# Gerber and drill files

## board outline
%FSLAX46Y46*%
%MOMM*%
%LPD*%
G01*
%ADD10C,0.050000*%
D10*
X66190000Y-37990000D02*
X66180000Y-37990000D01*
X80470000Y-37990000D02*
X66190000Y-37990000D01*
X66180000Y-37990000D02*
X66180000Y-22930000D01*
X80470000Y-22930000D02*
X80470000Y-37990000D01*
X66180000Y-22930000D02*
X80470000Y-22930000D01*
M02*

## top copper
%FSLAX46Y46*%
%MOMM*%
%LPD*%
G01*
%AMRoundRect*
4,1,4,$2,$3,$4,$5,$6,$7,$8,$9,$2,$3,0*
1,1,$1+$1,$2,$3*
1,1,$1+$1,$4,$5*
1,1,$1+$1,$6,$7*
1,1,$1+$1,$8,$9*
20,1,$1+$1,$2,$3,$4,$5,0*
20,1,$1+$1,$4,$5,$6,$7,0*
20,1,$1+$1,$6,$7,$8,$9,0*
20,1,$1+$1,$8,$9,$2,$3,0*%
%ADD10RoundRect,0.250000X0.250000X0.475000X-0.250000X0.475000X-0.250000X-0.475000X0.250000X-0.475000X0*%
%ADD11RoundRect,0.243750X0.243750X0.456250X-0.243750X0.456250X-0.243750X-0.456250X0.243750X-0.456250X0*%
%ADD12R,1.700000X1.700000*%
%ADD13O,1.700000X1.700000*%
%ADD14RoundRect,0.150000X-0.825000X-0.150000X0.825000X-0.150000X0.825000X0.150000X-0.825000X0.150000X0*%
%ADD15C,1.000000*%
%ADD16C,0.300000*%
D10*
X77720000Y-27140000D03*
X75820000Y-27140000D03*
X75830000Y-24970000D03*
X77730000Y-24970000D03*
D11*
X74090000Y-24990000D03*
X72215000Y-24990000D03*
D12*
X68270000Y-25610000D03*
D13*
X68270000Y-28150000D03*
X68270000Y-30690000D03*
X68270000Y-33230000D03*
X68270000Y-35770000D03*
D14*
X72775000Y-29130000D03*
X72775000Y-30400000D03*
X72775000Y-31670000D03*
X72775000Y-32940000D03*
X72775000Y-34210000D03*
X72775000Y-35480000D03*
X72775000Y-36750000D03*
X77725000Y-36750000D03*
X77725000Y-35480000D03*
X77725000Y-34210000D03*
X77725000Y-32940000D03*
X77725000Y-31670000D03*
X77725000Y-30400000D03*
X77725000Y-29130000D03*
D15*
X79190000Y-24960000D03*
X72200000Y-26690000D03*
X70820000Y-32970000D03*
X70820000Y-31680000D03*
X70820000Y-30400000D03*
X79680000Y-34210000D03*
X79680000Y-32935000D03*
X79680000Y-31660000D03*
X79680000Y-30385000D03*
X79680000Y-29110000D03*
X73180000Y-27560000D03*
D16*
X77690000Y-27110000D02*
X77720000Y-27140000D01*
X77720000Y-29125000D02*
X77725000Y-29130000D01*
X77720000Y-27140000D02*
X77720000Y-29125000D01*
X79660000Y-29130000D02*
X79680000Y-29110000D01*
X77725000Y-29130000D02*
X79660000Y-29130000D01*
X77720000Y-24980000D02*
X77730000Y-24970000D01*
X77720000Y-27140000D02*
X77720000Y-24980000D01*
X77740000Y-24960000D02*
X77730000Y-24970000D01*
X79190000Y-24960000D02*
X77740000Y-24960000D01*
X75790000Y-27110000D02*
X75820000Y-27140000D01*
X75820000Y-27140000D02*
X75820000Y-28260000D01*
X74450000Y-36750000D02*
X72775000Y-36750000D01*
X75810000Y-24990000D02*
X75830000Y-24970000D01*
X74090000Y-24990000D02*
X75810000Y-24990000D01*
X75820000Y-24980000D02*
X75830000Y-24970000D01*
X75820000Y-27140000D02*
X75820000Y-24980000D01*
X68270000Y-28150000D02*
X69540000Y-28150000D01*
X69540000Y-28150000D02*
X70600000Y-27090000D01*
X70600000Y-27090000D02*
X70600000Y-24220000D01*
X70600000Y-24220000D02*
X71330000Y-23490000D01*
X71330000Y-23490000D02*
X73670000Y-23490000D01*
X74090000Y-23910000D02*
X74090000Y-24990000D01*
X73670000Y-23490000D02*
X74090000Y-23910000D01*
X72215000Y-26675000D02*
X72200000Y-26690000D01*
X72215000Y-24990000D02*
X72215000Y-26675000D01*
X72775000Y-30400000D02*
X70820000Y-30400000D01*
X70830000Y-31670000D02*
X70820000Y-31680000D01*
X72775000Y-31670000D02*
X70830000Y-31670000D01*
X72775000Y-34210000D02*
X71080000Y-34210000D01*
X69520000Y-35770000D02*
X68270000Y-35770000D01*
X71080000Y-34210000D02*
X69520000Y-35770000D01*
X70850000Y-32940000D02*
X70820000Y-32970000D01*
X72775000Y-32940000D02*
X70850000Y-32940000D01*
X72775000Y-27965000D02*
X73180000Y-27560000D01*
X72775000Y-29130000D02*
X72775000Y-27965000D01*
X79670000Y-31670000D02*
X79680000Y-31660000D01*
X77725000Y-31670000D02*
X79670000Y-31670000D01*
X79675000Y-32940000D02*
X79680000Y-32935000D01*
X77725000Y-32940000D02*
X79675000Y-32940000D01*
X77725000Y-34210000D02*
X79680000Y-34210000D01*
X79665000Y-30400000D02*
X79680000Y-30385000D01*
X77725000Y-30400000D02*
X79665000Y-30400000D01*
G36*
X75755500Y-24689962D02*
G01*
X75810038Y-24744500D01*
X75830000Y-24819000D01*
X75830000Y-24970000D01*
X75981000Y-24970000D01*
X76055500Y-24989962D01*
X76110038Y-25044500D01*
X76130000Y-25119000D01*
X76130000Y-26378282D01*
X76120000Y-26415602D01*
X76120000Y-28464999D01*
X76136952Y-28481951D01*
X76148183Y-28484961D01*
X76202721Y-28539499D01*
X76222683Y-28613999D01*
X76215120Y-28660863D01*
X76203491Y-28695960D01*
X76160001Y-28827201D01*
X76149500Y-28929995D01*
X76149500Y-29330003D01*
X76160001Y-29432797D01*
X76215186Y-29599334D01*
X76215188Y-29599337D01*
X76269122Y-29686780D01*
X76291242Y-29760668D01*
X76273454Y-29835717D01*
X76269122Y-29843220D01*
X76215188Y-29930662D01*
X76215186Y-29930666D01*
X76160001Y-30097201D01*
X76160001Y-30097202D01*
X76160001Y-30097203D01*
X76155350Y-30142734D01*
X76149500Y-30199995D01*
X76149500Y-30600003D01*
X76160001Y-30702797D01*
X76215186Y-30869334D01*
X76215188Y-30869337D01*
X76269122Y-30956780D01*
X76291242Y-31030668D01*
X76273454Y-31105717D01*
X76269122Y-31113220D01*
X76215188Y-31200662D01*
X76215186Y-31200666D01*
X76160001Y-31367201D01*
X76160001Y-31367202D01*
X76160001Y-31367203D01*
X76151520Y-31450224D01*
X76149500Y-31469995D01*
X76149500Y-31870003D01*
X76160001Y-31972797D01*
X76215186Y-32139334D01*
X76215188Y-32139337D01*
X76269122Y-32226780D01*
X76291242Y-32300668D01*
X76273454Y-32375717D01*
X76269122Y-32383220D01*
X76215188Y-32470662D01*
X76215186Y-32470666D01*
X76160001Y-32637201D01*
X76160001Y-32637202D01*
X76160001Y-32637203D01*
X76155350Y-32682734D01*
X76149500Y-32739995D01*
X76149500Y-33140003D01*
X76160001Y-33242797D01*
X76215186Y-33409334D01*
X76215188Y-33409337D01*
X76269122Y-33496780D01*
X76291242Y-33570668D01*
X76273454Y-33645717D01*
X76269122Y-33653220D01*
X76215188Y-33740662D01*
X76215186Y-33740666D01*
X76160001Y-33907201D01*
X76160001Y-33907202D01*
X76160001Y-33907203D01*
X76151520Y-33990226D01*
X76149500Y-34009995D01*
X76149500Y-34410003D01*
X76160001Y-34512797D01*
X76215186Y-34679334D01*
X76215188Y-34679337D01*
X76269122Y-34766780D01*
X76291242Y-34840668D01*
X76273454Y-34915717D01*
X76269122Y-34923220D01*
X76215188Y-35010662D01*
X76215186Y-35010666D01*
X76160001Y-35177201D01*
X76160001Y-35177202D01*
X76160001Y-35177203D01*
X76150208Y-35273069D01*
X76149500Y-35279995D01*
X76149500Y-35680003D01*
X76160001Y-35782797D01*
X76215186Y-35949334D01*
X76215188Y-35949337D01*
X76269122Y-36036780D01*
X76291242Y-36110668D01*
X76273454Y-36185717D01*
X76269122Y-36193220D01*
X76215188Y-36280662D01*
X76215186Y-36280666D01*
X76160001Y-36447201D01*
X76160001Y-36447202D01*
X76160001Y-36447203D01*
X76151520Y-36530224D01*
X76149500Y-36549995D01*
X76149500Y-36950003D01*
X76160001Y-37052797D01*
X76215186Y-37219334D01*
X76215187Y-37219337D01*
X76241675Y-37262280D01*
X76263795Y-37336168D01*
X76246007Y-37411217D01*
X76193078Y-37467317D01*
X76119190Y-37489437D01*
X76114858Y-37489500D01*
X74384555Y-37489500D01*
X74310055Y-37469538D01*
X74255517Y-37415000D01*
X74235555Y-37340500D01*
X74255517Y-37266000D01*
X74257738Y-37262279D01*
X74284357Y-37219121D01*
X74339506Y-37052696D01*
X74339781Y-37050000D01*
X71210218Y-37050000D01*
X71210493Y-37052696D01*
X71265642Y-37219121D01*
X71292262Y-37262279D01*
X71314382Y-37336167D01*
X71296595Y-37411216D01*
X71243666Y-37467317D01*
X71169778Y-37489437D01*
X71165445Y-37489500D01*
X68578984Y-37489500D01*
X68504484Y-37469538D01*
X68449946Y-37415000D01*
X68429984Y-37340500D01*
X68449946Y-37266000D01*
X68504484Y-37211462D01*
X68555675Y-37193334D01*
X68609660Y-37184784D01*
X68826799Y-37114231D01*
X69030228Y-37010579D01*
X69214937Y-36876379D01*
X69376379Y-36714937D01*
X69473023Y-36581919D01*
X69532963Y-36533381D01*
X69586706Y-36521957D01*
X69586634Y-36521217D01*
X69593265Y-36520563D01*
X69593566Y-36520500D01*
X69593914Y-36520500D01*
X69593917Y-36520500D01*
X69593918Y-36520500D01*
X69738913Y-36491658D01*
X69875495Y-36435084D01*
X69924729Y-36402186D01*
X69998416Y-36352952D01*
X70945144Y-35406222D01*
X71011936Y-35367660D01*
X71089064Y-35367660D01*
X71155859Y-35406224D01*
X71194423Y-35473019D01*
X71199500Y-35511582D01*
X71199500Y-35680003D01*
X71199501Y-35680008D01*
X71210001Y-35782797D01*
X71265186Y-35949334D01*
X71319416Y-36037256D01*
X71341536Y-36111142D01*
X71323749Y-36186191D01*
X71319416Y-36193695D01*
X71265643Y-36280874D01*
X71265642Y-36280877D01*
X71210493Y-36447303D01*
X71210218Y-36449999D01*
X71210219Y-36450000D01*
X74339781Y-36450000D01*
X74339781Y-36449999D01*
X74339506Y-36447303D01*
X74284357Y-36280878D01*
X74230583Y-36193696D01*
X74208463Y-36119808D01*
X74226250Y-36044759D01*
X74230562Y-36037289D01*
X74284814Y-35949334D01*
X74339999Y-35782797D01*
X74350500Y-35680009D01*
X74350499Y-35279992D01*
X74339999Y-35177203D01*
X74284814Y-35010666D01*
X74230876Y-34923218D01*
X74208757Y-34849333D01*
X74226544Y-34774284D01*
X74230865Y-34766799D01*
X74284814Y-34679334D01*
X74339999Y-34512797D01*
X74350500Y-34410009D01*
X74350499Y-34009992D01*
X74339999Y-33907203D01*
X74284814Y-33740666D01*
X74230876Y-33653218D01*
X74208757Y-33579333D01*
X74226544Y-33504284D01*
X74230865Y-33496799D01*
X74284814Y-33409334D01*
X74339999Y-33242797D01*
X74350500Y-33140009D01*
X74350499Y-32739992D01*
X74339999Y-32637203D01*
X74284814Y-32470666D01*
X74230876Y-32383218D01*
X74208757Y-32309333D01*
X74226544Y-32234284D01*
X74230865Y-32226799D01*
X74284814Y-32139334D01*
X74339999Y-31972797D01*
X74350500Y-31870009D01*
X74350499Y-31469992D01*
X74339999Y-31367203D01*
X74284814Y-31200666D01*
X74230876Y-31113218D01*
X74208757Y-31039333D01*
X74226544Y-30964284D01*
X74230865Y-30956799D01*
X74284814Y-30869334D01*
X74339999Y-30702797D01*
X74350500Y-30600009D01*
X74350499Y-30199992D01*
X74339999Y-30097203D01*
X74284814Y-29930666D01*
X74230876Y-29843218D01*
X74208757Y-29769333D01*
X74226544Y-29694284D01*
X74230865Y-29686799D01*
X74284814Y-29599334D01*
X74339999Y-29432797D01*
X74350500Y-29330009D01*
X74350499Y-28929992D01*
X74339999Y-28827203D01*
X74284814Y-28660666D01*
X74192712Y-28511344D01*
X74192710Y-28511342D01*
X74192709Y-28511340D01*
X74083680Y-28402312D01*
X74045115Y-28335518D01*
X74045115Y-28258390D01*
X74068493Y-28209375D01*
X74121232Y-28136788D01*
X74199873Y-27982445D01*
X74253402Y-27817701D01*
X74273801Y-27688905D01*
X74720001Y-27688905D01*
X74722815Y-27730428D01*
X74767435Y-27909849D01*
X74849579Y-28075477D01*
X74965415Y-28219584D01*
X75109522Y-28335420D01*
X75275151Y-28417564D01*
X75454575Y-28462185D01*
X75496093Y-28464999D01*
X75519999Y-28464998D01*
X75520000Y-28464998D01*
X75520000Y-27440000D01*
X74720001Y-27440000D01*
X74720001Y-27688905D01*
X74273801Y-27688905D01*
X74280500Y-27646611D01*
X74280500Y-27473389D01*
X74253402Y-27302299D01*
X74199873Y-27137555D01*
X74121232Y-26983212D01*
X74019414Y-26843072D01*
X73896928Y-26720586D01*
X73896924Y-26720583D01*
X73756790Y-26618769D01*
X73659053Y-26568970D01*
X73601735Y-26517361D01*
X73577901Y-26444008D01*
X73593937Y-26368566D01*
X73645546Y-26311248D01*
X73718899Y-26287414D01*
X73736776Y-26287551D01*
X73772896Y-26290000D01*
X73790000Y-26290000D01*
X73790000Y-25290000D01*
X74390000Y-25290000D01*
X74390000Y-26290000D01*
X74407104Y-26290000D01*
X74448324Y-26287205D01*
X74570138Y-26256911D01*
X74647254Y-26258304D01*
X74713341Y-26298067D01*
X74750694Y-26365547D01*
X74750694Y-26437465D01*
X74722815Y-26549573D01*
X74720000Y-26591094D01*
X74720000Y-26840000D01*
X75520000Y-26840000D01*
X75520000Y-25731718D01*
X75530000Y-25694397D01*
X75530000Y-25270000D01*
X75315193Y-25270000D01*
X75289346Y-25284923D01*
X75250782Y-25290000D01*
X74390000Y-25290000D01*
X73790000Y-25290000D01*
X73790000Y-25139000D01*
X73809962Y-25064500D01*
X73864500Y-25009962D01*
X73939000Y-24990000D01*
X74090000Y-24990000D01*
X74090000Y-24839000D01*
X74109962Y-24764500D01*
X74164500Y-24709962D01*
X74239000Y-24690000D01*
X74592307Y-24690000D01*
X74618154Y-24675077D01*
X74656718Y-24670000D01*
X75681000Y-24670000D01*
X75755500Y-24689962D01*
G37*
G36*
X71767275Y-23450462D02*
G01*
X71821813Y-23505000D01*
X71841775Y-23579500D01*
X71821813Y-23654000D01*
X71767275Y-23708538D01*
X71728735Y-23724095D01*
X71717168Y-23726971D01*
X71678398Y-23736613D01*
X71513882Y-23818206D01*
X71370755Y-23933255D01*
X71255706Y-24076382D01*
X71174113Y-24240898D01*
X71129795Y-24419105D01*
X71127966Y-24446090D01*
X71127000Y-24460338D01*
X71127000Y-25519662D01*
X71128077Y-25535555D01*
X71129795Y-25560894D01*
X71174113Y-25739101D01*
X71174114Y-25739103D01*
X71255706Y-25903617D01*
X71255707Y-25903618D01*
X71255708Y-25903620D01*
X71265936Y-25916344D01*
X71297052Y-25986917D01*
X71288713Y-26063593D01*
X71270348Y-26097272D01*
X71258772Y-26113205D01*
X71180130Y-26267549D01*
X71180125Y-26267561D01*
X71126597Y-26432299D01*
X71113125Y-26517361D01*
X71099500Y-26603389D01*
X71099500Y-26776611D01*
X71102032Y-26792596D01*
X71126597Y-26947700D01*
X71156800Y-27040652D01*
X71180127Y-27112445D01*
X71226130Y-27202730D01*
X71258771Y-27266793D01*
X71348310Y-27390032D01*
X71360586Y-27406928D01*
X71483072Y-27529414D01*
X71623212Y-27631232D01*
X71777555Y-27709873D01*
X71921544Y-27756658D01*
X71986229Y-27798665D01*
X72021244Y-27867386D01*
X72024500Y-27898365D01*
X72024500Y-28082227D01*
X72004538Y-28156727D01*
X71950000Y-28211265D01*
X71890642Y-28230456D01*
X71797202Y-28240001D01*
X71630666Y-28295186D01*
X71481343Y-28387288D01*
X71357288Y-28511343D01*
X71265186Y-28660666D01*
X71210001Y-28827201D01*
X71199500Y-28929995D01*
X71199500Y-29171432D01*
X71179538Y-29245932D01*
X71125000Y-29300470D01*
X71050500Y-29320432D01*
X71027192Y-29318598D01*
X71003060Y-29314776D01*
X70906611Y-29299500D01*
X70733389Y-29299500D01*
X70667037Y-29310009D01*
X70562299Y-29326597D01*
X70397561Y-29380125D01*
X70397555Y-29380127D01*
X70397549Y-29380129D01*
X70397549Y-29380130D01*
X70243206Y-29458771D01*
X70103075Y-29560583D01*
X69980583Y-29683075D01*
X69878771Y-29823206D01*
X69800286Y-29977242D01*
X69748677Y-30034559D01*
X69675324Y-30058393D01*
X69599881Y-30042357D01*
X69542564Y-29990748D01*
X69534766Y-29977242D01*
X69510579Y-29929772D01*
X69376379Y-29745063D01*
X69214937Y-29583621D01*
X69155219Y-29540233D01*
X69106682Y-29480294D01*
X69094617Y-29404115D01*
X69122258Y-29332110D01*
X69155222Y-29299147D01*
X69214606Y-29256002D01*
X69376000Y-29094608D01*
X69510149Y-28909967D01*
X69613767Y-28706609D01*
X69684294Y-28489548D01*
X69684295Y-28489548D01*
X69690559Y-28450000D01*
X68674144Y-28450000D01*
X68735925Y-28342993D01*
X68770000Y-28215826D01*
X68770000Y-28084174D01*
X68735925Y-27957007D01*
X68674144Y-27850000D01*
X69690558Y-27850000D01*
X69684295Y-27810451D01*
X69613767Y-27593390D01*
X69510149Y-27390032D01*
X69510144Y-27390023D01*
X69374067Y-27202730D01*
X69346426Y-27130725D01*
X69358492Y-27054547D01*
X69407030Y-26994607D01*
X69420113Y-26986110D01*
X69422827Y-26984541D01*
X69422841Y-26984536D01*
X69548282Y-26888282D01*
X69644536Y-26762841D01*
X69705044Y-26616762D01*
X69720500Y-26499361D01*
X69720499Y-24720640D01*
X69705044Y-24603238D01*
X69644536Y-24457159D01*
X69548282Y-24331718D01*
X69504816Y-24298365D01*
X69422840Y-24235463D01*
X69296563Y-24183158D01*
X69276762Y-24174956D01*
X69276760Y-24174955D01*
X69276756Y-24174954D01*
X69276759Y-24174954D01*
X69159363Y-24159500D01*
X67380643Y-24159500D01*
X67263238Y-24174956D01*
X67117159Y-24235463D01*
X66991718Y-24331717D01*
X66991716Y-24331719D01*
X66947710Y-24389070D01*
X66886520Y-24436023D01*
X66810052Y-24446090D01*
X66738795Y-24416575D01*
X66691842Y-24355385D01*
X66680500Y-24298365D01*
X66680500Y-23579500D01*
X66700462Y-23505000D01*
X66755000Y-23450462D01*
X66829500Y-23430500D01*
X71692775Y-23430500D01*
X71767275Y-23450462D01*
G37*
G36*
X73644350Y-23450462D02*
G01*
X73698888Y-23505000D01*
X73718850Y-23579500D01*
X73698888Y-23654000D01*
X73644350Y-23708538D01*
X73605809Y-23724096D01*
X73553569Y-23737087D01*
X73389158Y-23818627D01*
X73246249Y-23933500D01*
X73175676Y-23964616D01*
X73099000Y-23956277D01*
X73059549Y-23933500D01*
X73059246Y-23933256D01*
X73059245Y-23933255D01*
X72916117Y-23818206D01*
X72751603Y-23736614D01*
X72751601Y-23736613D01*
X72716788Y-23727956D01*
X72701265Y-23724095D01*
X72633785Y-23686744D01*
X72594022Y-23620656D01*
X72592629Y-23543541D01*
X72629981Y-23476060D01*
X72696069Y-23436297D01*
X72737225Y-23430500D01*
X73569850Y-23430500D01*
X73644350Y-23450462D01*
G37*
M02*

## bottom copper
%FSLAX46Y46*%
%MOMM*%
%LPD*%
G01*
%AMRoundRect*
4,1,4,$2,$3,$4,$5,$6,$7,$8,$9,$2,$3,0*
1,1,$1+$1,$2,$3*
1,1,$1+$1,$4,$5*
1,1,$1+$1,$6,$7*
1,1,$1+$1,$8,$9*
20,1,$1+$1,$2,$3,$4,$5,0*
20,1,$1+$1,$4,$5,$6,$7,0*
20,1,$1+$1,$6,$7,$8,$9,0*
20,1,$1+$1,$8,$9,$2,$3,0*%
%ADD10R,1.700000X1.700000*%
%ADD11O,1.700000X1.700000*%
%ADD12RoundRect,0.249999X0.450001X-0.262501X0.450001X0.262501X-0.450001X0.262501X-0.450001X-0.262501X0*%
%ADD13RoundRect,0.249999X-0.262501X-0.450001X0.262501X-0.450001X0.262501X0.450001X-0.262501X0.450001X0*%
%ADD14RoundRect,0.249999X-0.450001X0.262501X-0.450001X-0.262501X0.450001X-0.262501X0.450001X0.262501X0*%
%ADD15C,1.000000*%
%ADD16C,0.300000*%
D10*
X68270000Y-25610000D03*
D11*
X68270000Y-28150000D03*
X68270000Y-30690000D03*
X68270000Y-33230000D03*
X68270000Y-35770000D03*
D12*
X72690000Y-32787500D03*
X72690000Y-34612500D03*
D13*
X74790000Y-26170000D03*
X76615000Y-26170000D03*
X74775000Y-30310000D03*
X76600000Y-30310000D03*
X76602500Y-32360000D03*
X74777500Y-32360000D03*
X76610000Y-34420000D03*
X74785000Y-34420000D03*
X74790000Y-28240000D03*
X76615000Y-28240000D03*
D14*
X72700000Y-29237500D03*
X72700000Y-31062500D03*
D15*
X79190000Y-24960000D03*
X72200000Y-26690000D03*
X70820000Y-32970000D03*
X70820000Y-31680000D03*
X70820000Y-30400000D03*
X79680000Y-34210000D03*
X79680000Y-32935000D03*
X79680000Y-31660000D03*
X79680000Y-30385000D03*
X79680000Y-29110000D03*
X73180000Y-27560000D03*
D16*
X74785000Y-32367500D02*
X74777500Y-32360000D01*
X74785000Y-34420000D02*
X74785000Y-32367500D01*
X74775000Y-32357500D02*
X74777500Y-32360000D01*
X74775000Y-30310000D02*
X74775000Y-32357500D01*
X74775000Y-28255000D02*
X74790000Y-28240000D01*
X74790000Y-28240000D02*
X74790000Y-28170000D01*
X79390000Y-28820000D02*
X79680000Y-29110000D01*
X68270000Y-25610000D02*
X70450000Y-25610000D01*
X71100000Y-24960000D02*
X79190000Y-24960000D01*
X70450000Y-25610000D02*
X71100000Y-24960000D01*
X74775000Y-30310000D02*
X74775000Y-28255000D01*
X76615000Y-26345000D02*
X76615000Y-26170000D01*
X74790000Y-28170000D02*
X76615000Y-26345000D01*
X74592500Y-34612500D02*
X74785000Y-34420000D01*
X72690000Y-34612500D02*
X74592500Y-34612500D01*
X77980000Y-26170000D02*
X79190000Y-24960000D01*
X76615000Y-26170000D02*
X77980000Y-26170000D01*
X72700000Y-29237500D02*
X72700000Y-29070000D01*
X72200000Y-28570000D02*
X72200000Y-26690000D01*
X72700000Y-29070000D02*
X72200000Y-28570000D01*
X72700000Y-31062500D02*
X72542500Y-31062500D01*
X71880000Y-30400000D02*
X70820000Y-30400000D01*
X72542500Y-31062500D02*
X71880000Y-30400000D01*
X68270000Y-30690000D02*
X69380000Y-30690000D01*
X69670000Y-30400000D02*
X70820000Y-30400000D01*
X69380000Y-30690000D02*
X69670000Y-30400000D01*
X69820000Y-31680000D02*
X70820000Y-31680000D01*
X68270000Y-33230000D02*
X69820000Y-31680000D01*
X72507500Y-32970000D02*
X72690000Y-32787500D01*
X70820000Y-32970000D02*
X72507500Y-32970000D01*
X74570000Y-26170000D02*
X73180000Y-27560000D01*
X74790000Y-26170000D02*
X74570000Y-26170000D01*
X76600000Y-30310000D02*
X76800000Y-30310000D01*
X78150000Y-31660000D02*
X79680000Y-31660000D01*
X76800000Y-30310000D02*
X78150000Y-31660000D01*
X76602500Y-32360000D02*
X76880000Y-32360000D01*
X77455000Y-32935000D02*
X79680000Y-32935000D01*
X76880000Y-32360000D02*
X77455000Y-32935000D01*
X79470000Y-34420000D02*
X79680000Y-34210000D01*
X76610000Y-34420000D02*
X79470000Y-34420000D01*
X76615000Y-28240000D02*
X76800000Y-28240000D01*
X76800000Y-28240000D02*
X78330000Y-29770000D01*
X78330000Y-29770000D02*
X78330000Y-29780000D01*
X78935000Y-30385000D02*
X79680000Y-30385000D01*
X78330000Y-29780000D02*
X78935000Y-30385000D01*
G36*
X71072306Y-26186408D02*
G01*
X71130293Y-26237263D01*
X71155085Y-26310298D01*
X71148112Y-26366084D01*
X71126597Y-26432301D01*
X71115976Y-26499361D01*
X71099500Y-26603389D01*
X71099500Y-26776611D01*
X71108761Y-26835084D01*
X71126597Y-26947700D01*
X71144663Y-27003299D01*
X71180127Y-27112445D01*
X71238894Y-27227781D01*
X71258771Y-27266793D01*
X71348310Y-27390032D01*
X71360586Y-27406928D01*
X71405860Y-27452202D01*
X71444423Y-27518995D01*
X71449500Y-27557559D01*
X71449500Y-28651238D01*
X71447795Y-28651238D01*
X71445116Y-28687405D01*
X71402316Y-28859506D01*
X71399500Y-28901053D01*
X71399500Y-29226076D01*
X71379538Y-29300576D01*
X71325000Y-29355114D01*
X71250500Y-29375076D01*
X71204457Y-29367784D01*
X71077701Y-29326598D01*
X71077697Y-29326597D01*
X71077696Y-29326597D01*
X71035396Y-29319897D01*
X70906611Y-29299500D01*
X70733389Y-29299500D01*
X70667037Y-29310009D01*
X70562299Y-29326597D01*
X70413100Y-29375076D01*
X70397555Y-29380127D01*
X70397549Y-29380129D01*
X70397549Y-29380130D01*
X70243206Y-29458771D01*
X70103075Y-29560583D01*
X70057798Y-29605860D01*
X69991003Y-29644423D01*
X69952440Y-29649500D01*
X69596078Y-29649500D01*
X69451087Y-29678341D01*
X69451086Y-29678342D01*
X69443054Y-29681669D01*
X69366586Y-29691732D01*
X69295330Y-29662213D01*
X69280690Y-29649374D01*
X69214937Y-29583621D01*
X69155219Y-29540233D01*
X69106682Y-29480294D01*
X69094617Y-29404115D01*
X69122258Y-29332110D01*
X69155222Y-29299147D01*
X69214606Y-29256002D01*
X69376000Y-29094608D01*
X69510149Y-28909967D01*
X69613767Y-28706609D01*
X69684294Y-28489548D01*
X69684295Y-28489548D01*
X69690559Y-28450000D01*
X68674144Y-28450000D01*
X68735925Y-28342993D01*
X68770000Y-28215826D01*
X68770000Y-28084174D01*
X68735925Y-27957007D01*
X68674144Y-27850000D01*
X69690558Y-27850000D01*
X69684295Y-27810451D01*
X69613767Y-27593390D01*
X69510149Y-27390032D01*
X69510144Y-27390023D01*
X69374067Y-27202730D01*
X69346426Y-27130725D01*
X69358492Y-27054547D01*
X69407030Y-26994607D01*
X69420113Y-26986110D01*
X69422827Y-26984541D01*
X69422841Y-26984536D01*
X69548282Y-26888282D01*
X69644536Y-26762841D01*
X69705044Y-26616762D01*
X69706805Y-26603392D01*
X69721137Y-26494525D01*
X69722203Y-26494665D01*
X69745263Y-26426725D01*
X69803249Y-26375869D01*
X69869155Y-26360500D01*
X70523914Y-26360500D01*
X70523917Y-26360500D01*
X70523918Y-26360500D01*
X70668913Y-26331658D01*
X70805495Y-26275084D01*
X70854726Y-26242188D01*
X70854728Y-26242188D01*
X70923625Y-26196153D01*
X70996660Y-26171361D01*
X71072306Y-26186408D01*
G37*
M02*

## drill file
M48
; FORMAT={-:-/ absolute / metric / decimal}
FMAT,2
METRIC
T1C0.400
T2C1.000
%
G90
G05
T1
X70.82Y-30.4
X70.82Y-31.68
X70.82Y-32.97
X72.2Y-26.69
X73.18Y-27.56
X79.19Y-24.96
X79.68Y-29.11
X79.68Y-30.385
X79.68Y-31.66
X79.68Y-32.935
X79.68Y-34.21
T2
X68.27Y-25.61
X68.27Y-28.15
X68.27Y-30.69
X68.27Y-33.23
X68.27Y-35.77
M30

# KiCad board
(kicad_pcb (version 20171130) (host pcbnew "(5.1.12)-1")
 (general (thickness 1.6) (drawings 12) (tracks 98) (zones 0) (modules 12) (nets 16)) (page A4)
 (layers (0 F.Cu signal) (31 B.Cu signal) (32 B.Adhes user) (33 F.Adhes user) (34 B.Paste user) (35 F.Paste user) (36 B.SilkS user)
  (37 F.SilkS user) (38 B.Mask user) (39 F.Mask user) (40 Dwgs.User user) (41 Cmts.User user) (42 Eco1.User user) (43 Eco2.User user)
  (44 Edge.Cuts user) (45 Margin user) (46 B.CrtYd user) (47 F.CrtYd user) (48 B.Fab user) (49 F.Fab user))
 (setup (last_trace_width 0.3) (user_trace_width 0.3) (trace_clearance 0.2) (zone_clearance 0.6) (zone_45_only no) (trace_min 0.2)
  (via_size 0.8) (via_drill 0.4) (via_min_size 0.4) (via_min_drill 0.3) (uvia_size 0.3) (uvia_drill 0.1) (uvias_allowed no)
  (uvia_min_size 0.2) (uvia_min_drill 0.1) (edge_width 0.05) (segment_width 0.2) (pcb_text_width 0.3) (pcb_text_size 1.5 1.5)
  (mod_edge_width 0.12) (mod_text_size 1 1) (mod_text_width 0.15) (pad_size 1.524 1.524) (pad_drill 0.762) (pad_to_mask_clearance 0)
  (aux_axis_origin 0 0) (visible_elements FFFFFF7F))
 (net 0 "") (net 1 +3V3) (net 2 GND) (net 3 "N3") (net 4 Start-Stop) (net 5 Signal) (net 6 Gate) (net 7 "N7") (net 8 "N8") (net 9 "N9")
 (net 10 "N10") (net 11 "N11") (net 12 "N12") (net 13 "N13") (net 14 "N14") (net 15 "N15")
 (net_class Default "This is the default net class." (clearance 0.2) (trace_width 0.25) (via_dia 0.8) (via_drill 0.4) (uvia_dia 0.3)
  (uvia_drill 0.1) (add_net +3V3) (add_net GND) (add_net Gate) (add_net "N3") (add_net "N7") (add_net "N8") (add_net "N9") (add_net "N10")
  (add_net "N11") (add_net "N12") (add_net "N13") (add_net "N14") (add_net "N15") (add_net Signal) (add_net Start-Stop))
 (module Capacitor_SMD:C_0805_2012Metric (layer F.Cu) (at 76.77 27.14 180)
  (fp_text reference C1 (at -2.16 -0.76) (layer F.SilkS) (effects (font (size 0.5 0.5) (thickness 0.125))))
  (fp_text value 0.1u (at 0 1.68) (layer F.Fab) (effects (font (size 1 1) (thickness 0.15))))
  (pad 1 smd roundrect (at -0.95 0 180) (size 1 1.45) (layers F.Cu F.Paste F.Mask) (roundrect_rratio 0.25) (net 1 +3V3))
  (pad 2 smd roundrect (at 0.95 0 180) (size 1 1.45) (layers F.Cu F.Paste F.Mask) (roundrect_rratio 0.25) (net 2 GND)))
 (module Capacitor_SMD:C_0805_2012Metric (layer F.Cu) (at 76.78 24.97 180)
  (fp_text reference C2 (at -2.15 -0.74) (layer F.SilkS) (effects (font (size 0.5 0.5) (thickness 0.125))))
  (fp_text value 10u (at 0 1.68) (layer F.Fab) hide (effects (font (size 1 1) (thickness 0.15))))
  (pad 2 smd roundrect (at 0.95 0 180) (size 1 1.45) (layers F.Cu F.Paste F.Mask) (roundrect_rratio 0.25) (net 2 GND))
  (pad 1 smd roundrect (at -0.95 0 180) (size 1 1.45) (layers F.Cu F.Paste F.Mask) (roundrect_rratio 0.25) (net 1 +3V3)))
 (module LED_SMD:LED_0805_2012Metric (layer F.Cu) (at 73.1525 24.99 180)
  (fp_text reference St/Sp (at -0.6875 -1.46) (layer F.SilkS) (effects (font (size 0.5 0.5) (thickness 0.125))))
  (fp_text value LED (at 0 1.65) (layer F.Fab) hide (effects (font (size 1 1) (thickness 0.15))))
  (pad 1 smd roundrect (at -0.9375 0 180) (size 0.975 1.4) (layers F.Cu F.Paste F.Mask) (roundrect_rratio 0.25) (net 2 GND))
  (pad 2 smd roundrect (at 0.9375 0 180) (size 0.975 1.4) (layers F.Cu F.Paste F.Mask) (roundrect_rratio 0.25) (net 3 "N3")))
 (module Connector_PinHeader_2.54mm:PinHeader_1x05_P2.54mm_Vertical (layer F.Cu) (at 68.27 25.61)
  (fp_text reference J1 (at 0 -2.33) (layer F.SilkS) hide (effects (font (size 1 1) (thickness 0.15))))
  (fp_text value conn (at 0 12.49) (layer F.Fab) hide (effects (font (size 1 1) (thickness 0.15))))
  (pad 1 thru_hole rect (at 0 0) (size 1.7 1.7) (drill 1) (layers *.Cu *.Mask) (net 1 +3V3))
  (pad 2 thru_hole oval (at 0 2.54) (size 1.7 1.7) (drill 1) (layers *.Cu *.Mask) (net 2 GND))
  (pad 3 thru_hole oval (at 0 5.08) (size 1.7 1.7) (drill 1) (layers *.Cu *.Mask) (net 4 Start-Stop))
  (pad 4 thru_hole oval (at 0 7.62) (size 1.7 1.7) (drill 1) (layers *.Cu *.Mask) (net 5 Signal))
  (pad 5 thru_hole oval (at 0 10.16) (size 1.7 1.7) (drill 1) (layers *.Cu *.Mask) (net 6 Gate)))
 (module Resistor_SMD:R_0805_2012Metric (layer B.Cu) (at 72.69 33.7 90)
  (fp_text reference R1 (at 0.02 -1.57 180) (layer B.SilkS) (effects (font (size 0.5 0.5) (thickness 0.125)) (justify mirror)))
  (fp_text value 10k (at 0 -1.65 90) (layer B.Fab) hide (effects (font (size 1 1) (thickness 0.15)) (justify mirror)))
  (pad 2 smd roundrect (at 0.9125 0 90) (size 1.025 1.4) (layers B.Cu B.Paste B.Mask) (roundrect_rratio 0.2439014634146341) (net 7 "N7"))
  (pad 1 smd roundrect (at -0.9125 0 90) (size 1.025 1.4) (layers B.Cu B.Paste B.Mask) (roundrect_rratio 0.2439014634146341) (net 1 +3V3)))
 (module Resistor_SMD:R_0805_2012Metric (layer B.Cu) (at 75.7025 26.17)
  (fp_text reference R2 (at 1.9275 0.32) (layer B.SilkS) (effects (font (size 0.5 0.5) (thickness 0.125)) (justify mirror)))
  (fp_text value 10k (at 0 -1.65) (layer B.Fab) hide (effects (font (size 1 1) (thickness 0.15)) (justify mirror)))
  (pad 1 smd roundrect (at -0.9125 0) (size 1.025 1.4) (layers B.Cu B.Paste B.Mask) (roundrect_rratio 0.2439014634146341) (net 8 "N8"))
  (pad 2 smd roundrect (at 0.9125 0) (size 1.025 1.4) (layers B.Cu B.Paste B.Mask) (roundrect_rratio 0.2439014634146341) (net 1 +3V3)))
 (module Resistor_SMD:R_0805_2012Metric (layer B.Cu) (at 75.6875 30.31)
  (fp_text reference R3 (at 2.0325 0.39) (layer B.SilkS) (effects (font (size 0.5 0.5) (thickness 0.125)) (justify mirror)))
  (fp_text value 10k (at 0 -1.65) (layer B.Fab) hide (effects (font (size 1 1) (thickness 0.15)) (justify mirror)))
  (pad 1 smd roundrect (at -0.9125 0) (size 1.025 1.4) (layers B.Cu B.Paste B.Mask) (roundrect_rratio 0.2439014634146341) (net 1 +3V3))
  (pad 2 smd roundrect (at 0.9125 0) (size 1.025 1.4) (layers B.Cu B.Paste B.Mask) (roundrect_rratio 0.2439014634146341) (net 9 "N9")))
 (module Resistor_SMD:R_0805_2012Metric (layer B.Cu) (at 75.69 32.36)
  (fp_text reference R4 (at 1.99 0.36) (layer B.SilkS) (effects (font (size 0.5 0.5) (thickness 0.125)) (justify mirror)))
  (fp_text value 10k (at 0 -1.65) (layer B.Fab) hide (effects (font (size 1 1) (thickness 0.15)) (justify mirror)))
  (pad 2 smd roundrect (at 0.9125 0) (size 1.025 1.4) (layers B.Cu B.Paste B.Mask) (roundrect_rratio 0.2439014634146341) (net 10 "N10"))
  (pad 1 smd roundrect (at -0.9125 0) (size 1.025 1.4) (layers B.Cu B.Paste B.Mask) (roundrect_rratio 0.2439014634146341) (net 1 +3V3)))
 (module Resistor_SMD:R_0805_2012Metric (layer B.Cu) (at 75.6975 34.42)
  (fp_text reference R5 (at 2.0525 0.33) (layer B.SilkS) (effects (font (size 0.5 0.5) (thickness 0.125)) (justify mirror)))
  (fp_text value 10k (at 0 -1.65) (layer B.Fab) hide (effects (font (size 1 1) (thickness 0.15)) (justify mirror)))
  (pad 2 smd roundrect (at 0.9125 0) (size 1.025 1.4) (layers B.Cu B.Paste B.Mask) (roundrect_rratio 0.2439014634146341) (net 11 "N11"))
  (pad 1 smd roundrect (at -0.9125 0) (size 1.025 1.4) (layers B.Cu B.Paste B.Mask) (roundrect_rratio 0.2439014634146341) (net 1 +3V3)))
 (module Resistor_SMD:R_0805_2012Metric (layer B.Cu) (at 75.7025 28.24)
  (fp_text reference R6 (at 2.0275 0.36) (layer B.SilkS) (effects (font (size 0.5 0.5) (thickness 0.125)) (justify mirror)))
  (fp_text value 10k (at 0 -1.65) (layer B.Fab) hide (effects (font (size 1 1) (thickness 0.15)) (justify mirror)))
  (pad 1 smd roundrect (at -0.9125 0) (size 1.025 1.4) (layers B.Cu B.Paste B.Mask) (roundrect_rratio 0.2439014634146341) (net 1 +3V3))
  (pad 2 smd roundrect (at 0.9125 0) (size 1.025 1.4) (layers B.Cu B.Paste B.Mask) (roundrect_rratio 0.2439014634146341) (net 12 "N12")))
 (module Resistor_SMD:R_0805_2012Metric (layer B.Cu) (at 72.7 30.15 270)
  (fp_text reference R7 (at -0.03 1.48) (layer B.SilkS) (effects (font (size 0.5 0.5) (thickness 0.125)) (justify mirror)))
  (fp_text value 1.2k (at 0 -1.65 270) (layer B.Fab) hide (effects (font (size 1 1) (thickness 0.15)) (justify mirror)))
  (pad 1 smd roundrect (at -0.9125 0 270) (size 1.025 1.4) (layers B.Cu B.Paste B.Mask) (roundrect_rratio 0.2439014634146341) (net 3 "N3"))
  (pad 2 smd roundrect (at 0.9125 0 270) (size 1.025 1.4) (layers B.Cu B.Paste B.Mask) (roundrect_rratio 0.2439014634146341)
   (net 4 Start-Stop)))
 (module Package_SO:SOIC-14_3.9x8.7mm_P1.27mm (layer F.Cu) (at 75.25 32.94)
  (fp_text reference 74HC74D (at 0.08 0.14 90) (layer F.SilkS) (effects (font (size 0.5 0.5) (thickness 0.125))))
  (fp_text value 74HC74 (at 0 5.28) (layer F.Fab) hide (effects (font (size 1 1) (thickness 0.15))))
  (pad 1 smd roundrect (at -2.475 -3.81) (size 1.95 0.6) (layers F.Cu F.Paste F.Mask) (roundrect_rratio 0.25) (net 8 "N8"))
  (pad 2 smd roundrect (at -2.475 -2.54) (size 1.95 0.6) (layers F.Cu F.Paste F.Mask) (roundrect_rratio 0.25) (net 4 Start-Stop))
  (pad 3 smd roundrect (at -2.475 -1.27) (size 1.95 0.6) (layers F.Cu F.Paste F.Mask) (roundrect_rratio 0.25) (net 5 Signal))
  (pad 4 smd roundrect (at -2.475 0) (size 1.95 0.6) (layers F.Cu F.Paste F.Mask) (roundrect_rratio 0.25) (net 7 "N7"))
  (pad 5 smd roundrect (at -2.475 1.27) (size 1.95 0.6) (layers F.Cu F.Paste F.Mask) (roundrect_rratio 0.25) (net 6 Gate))
  (pad 6 smd roundrect (at -2.475 2.54) (size 1.95 0.6) (layers F.Cu F.Paste F.Mask) (roundrect_rratio 0.25) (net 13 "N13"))
  (pad 7 smd roundrect (at -2.475 3.81) (size 1.95 0.6) (layers F.Cu F.Paste F.Mask) (roundrect_rratio 0.25) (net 2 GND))
  (pad 8 smd roundrect (at 2.475 3.81) (size 1.95 0.6) (layers F.Cu F.Paste F.Mask) (roundrect_rratio 0.25) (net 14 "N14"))
  (pad 9 smd roundrect (at 2.475 2.54) (size 1.95 0.6) (layers F.Cu F.Paste F.Mask) (roundrect_rratio 0.25) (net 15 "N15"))
  (pad 10 smd roundrect (at 2.475 1.27) (size 1.95 0.6) (layers F.Cu F.Paste F.Mask) (roundrect_rratio 0.25) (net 11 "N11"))
  (pad 11 smd roundrect (at 2.475 0) (size 1.95 0.6) (layers F.Cu F.Paste F.Mask) (roundrect_rratio 0.25) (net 10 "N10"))
  (pad 12 smd roundrect (at 2.475 -1.27) (size 1.95 0.6) (layers F.Cu F.Paste F.Mask) (roundrect_rratio 0.25) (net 9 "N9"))
  (pad 13 smd roundrect (at 2.475 -2.54) (size 1.95 0.6) (layers F.Cu F.Paste F.Mask) (roundrect_rratio 0.25) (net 12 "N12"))
  (pad 14 smd roundrect (at 2.475 -3.81) (size 1.95 0.6) (layers F.Cu F.Paste F.Mask) (roundrect_rratio 0.25) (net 1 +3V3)))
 (gr_line (start 66.19 37.99) (end 66.18 37.99) (layer Edge.Cuts) (width 0.05))
 (gr_line (start 80.47 37.99) (end 66.19 37.99) (layer Edge.Cuts) (width 0.05))
 (gr_line (start 66.18 37.99) (end 66.18 22.93) (layer Edge.Cuts) (width 0.05))
 (gr_line (start 80.47 22.93) (end 80.47 37.99) (layer Edge.Cuts) (width 0.05))
 (gr_line (start 66.18 22.93) (end 80.47 22.93) (layer Edge.Cuts) (width 0.05))
 (via (at 79.19 24.96) (size 1) (drill 0.4) (layers F.Cu B.Cu) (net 1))
 (via (at 72.2 26.69) (size 1) (drill 0.4) (layers F.Cu B.Cu) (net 3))
 (via (at 70.82 32.97) (size 1) (drill 0.4) (layers F.Cu B.Cu) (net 7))
 (via (at 70.82 31.68) (size 1) (drill 0.4) (layers F.Cu B.Cu) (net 5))
 (via (at 70.82 30.4) (size 1) (drill 0.4) (layers F.Cu B.Cu) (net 4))
 (via (at 79.68 34.21) (size 1) (drill 0.4) (layers F.Cu B.Cu) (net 11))
 (via (at 79.68 32.935) (size 1) (drill 0.4) (layers F.Cu B.Cu) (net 10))
 (via (at 79.68 31.66) (size 1) (drill 0.4) (layers F.Cu B.Cu) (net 9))
 (via (at 79.68 30.385) (size 1) (drill 0.4) (layers F.Cu B.Cu) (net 12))
 (via (at 79.68 29.11) (size 1) (drill 0.4) (layers F.Cu B.Cu) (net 1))
 (via (at 73.18 27.56) (size 1) (drill 0.4) (layers F.Cu B.Cu) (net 8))
 (segment (start 77.69 27.11) (end 77.72 27.14) (width 0.3) (layer F.Cu) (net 1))
 (segment (start 77.72 29.125) (end 77.725 29.13) (width 0.3) (layer F.Cu) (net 1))
 (segment (start 77.72 27.14) (end 77.72 29.125) (width 0.3) (layer F.Cu) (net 1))
 (segment (start 74.785 32.3675) (end 74.7775 32.36) (width 0.3) (layer B.Cu) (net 1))
 (segment (start 74.785 34.42) (end 74.785 32.3675) (width 0.3) (layer B.Cu) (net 1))
 (segment (start 74.775 32.3575) (end 74.7775 32.36) (width 0.3) (layer B.Cu) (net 1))
 (segment (start 74.775 30.31) (end 74.775 32.3575) (width 0.3) (layer B.Cu) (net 1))
 (segment (start 74.775 28.255) (end 74.79 28.24) (width 0.3) (layer B.Cu) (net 1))
 (segment (start 74.79 28.24) (end 74.79 28.17) (width 0.3) (layer B.Cu) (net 1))
 (segment (start 79.66 29.13) (end 79.68 29.11) (width 0.3) (layer F.Cu) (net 1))
 (segment (start 77.725 29.13) (end 79.66 29.13) (width 0.3) (layer F.Cu) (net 1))
 (segment (start 79.39 28.82) (end 79.68 29.11) (width 0.3) (layer B.Cu) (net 1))
 (segment (start 77.72 24.98) (end 77.73 24.97) (width 0.3) (layer F.Cu) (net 1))
 (segment (start 77.72 27.14) (end 77.72 24.98) (width 0.3) (layer F.Cu) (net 1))
 (segment (start 77.74 24.96) (end 77.73 24.97) (width 0.3) (layer F.Cu) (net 1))
 (segment (start 79.19 24.96) (end 77.74 24.96) (width 0.3) (layer F.Cu) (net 1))
 (segment (start 68.27 25.61) (end 70.45 25.61) (width 0.3) (layer B.Cu) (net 1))
 (segment (start 71.1 24.96) (end 79.19 24.96) (width 0.3) (layer B.Cu) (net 1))
 (segment (start 70.45 25.61) (end 71.1 24.96) (width 0.3) (layer B.Cu) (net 1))
 (segment (start 74.775 30.31) (end 74.775 28.255) (width 0.3) (layer B.Cu) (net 1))
 (segment (start 76.615 26.345) (end 76.615 26.17) (width 0.3) (layer B.Cu) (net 1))
 (segment (start 74.79 28.17) (end 76.615 26.345) (width 0.3) (layer B.Cu) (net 1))
 (segment (start 74.5925 34.6125) (end 74.785 34.42) (width 0.3) (layer B.Cu) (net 1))
 (segment (start 72.69 34.6125) (end 74.5925 34.6125) (width 0.3) (layer B.Cu) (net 1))
 (segment (start 77.98 26.17) (end 79.19 24.96) (width 0.3) (layer B.Cu) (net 1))
 (segment (start 76.615 26.17) (end 77.98 26.17) (width 0.3) (layer B.Cu) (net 1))
 (segment (start 75.79 27.11) (end 75.82 27.14) (width 0.3) (layer F.Cu) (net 2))
 (segment (start 75.82 27.14) (end 75.82 28.26) (width 0.3) (layer F.Cu) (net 2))
 (segment (start 74.45 36.75) (end 72.775 36.75) (width 0.3) (layer F.Cu) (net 2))
 (segment (start 75.81 24.99) (end 75.83 24.97) (width 0.3) (layer F.Cu) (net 2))
 (segment (start 74.09 24.99) (end 75.81 24.99) (width 0.3) (layer F.Cu) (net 2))
 (segment (start 75.82 24.98) (end 75.83 24.97) (width 0.3) (layer F.Cu) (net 2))
 (segment (start 75.82 27.14) (end 75.82 24.98) (width 0.3) (layer F.Cu) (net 2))
 (segment (start 68.27 28.15) (end 69.54 28.15) (width 0.3) (layer F.Cu) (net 2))
 (segment (start 69.54 28.15) (end 70.6 27.09) (width 0.3) (layer F.Cu) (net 2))
 (segment (start 70.6 27.09) (end 70.6 24.22) (width 0.3) (layer F.Cu) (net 2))
 (segment (start 70.6 24.22) (end 71.33 23.49) (width 0.3) (layer F.Cu) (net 2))
 (segment (start 71.33 23.49) (end 73.67 23.49) (width 0.3) (layer F.Cu) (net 2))
 (segment (start 74.09 23.91) (end 74.09 24.99) (width 0.3) (layer F.Cu) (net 2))
 (segment (start 73.67 23.49) (end 74.09 23.91) (width 0.3) (layer F.Cu) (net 2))
 (segment (start 72.215 26.675) (end 72.2 26.69) (width 0.3) (layer F.Cu) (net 3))
 (segment (start 72.215 24.99) (end 72.215 26.675) (width 0.3) (layer F.Cu) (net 3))
 (segment (start 72.7 29.2375) (end 72.7 29.07) (width 0.3) (layer B.Cu) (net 3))
 (segment (start 72.2 28.57) (end 72.2 26.69) (width 0.3) (layer B.Cu) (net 3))
 (segment (start 72.7 29.07) (end 72.2 28.57) (width 0.3) (layer B.Cu) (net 3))
 (segment (start 72.775 30.4) (end 70.82 30.4) (width 0.3) (layer F.Cu) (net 4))
 (segment (start 72.7 31.0625) (end 72.5425 31.0625) (width 0.3) (layer B.Cu) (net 4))
 (segment (start 71.88 30.4) (end 70.82 30.4) (width 0.3) (layer B.Cu) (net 4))
 (segment (start 72.5425 31.0625) (end 71.88 30.4) (width 0.3) (layer B.Cu) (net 4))
 (segment (start 68.27 30.69) (end 69.38 30.69) (width 0.3) (layer B.Cu) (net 4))
 (segment (start 69.67 30.4) (end 70.82 30.4) (width 0.3) (layer B.Cu) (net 4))
 (segment (start 69.38 30.69) (end 69.67 30.4) (width 0.3) (layer B.Cu) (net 4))
 (segment (start 70.83 31.67) (end 70.82 31.68) (width 0.3) (layer F.Cu) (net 5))
 (segment (start 72.775 31.67) (end 70.83 31.67) (width 0.3) (layer F.Cu) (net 5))
 (segment (start 69.82 31.68) (end 70.82 31.68) (width 0.3) (layer B.Cu) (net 5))
 (segment (start 68.27 33.23) (end 69.82 31.68) (width 0.3) (layer B.Cu) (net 5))
 (segment (start 72.775 34.21) (end 71.08 34.21) (width 0.3) (layer F.Cu) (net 6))
 (segment (start 69.52 35.77) (end 68.27 35.77) (width 0.3) (layer F.Cu) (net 6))
 (segment (start 71.08 34.21) (end 69.52 35.77) (width 0.3) (layer F.Cu) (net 6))
 (segment (start 70.85 32.94) (end 70.82 32.97) (width 0.3) (layer F.Cu) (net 7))
 (segment (start 72.775 32.94) (end 70.85 32.94) (width 0.3) (layer F.Cu) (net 7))
 (segment (start 72.5075 32.97) (end 72.69 32.7875) (width 0.3) (layer B.Cu) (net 7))
 (segment (start 70.82 32.97) (end 72.5075 32.97) (width 0.3) (layer B.Cu) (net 7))
 (segment (start 72.775 27.965) (end 73.18 27.56) (width 0.3) (layer F.Cu) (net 8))
 (segment (start 72.775 29.13) (end 72.775 27.965) (width 0.3) (layer F.Cu) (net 8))
 (segment (start 74.57 26.17) (end 73.18 27.56) (width 0.3) (layer B.Cu) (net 8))
 (segment (start 74.79 26.17) (end 74.57 26.17) (width 0.3) (layer B.Cu) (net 8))
 (segment (start 79.67 31.67) (end 79.68 31.66) (width 0.3) (layer F.Cu) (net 9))
 (segment (start 77.725 31.67) (end 79.67 31.67) (width 0.3) (layer F.Cu) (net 9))
 (segment (start 76.6 30.31) (end 76.8 30.31) (width 0.3) (layer B.Cu) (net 9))
 (segment (start 78.15 31.66) (end 79.68 31.66) (width 0.3) (layer B.Cu) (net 9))
 (segment (start 76.8 30.31) (end 78.15 31.66) (width 0.3) (layer B.Cu) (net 9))
 (segment (start 79.675 32.94) (end 79.68 32.935) (width 0.3) (layer F.Cu) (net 10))
 (segment (start 77.725 32.94) (end 79.675 32.94) (width 0.3) (layer F.Cu) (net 10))
 (segment (start 76.6025 32.36) (end 76.88 32.36) (width 0.3) (layer B.Cu) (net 10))
 (segment (start 77.455 32.935) (end 79.68 32.935) (width 0.3) (layer B.Cu) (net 10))
 (segment (start 76.88 32.36) (end 77.455 32.935) (width 0.3) (layer B.Cu) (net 10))
 (segment (start 77.725 34.21) (end 79.68 34.21) (width 0.3) (layer F.Cu) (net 11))
 (segment (start 79.47 34.42) (end 79.68 34.21) (width 0.3) (layer B.Cu) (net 11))
 (segment (start 76.61 34.42) (end 79.47 34.42) (width 0.3) (layer B.Cu) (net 11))
 (segment (start 79.665 30.4) (end 79.68 30.385) (width 0.3) (layer F.Cu) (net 12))
 (segment (start 77.725 30.4) (end 79.665 30.4) (width 0.3) (layer F.Cu) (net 12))
 (segment (start 76.615 28.24) (end 76.8 28.24) (width 0.3) (layer B.Cu) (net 12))
 (segment (start 76.8 28.24) (end 78.33 29.77) (width 0.3) (layer B.Cu) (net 12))
 (segment (start 78.33 29.77) (end 78.33 29.78) (width 0.3) (layer B.Cu) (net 12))
 (segment (start 78.935 30.385) (end 79.68 30.385) (width 0.3) (layer B.Cu) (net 12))
 (segment (start 78.33 29.78) (end 78.935 30.385) (width 0.3) (layer B.Cu) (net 12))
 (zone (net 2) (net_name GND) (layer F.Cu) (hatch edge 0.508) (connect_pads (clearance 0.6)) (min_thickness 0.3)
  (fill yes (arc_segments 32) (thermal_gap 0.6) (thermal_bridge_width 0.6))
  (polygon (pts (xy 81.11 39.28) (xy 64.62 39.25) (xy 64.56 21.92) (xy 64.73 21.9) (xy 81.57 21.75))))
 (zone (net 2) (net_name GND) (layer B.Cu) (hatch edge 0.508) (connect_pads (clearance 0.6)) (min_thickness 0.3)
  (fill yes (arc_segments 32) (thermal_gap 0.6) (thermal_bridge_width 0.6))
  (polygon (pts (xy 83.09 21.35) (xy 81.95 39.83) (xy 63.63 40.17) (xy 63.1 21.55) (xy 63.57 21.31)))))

